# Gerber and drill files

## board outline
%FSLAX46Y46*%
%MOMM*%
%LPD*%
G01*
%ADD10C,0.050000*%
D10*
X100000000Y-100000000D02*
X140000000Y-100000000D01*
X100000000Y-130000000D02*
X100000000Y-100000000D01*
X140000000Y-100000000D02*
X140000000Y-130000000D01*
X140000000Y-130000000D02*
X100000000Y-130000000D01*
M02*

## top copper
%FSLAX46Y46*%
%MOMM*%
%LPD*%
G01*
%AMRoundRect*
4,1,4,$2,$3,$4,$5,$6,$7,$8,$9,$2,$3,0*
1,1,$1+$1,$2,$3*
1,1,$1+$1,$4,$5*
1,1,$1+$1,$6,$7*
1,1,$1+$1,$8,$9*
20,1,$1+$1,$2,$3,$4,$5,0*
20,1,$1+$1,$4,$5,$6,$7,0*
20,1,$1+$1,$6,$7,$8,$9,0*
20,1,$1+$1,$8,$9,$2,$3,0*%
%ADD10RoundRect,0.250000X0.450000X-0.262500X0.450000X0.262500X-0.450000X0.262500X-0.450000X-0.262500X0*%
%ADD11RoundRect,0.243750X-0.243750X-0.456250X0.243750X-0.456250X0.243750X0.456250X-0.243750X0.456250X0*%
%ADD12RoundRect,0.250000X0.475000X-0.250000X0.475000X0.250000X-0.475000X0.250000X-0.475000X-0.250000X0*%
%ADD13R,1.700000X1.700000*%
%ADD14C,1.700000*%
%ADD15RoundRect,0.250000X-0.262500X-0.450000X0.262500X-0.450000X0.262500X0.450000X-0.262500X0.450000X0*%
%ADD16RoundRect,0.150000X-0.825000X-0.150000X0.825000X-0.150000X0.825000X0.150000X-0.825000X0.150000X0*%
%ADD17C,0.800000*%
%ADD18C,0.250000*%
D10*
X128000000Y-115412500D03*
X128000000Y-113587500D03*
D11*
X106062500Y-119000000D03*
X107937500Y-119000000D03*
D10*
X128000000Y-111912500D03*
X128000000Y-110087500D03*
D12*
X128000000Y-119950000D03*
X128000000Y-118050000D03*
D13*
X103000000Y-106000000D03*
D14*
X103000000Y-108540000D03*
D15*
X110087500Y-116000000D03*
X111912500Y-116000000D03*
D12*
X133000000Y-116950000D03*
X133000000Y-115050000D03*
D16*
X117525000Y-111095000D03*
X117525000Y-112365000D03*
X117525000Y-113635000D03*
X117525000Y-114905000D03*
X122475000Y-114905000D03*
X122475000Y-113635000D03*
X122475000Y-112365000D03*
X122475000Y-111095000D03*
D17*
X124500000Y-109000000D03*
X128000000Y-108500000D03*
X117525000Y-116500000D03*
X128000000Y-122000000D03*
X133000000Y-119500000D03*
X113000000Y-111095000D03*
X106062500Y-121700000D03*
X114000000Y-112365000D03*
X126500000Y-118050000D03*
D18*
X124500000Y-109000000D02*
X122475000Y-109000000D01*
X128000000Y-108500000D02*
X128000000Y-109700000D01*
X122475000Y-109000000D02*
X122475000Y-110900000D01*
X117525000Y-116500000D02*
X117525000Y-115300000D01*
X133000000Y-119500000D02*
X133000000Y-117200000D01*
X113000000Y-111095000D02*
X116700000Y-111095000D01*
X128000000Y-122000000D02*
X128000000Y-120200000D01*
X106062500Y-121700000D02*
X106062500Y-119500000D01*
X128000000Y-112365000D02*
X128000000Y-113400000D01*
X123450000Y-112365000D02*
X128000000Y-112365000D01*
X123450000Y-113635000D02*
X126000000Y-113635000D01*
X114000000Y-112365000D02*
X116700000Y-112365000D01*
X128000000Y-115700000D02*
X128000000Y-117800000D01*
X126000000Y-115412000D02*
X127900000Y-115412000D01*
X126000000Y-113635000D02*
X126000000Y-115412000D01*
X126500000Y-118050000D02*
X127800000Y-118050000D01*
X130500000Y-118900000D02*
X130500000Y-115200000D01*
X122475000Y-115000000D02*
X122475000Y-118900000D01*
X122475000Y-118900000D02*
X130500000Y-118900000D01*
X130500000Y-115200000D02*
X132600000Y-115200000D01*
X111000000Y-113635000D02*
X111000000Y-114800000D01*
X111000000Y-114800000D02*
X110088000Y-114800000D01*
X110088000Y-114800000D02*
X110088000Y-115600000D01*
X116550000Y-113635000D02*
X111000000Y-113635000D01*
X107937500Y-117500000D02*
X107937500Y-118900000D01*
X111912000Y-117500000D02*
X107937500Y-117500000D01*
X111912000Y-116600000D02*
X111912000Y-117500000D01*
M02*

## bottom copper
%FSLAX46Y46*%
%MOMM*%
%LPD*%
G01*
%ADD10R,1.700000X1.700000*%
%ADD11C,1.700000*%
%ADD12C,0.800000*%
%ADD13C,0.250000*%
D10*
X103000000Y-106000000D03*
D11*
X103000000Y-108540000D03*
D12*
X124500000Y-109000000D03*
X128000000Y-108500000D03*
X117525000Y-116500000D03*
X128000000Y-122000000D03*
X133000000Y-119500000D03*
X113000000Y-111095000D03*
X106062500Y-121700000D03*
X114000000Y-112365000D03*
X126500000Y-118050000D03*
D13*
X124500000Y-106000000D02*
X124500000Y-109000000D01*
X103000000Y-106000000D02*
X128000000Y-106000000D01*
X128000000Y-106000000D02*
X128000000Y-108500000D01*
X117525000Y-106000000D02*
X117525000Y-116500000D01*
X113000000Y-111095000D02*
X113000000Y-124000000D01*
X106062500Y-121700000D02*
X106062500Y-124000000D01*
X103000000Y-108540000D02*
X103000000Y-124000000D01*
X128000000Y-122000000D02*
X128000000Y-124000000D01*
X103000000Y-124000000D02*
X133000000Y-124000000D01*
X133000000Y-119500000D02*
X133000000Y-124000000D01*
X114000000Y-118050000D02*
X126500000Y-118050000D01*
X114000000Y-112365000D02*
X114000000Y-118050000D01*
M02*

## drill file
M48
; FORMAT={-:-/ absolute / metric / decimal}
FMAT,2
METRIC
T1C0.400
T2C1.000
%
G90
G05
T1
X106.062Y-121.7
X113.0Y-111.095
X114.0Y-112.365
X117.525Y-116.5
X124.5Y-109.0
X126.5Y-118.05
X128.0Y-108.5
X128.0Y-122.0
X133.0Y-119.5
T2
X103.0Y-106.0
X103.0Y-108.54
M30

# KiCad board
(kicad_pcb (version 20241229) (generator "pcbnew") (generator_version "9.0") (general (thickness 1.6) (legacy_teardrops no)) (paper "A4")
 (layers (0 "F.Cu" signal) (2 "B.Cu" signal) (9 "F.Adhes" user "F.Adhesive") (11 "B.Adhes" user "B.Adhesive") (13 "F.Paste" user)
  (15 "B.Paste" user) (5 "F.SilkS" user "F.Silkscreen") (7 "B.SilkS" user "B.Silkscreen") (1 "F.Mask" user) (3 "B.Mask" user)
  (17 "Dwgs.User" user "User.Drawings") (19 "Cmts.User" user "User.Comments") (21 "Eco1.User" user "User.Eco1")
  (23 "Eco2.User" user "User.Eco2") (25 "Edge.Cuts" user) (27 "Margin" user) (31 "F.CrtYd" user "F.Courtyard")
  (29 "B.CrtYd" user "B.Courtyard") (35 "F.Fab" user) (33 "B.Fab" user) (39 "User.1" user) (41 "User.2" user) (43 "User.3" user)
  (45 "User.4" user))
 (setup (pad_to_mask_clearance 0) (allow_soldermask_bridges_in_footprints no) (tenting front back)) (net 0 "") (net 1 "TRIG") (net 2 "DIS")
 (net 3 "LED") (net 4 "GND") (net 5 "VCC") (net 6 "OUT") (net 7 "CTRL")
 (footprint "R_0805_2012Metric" (layer "F.Cu") (at 128 114.5 90)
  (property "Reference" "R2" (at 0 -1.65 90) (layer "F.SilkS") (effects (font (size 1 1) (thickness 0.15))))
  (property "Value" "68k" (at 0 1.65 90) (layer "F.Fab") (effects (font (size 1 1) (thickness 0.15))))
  (pad "1" smd roundrect (at -0.9125 0 90) (size 1.025 1.4) (layers "F.Cu" "F.Mask" "F.Paste") (roundrect_rratio 0.243902) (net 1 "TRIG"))
  (pad "2" smd roundrect (at 0.9125 0 90) (size 1.025 1.4) (layers "F.Cu" "F.Mask" "F.Paste") (roundrect_rratio 0.243902) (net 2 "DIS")))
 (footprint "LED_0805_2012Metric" (layer "F.Cu") (at 107 119)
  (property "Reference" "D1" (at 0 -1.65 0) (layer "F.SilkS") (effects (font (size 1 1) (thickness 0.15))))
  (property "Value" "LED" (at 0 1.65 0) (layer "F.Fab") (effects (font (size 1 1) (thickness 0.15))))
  (pad "1" smd roundrect (at -0.9375 0) (size 0.975 1.4) (layers "F.Cu" "F.Mask" "F.Paste") (roundrect_rratio 0.25) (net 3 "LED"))
  (pad "2" smd roundrect (at 0.9375 0) (size 0.975 1.4) (layers "F.Cu" "F.Mask" "F.Paste") (roundrect_rratio 0.25) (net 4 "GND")))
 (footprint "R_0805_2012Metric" (layer "F.Cu") (at 128 111 90)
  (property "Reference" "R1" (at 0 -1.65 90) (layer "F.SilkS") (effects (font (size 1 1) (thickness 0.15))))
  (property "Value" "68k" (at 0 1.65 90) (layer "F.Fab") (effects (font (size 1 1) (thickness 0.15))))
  (pad "1" smd roundrect (at -0.9125 0 90) (size 1.025 1.4) (layers "F.Cu" "F.Mask" "F.Paste") (roundrect_rratio 0.243902) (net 2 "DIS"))
  (pad "2" smd roundrect (at 0.9125 0 90) (size 1.025 1.4) (layers "F.Cu" "F.Mask" "F.Paste") (roundrect_rratio 0.243902) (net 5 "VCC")))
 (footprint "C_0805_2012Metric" (layer "F.Cu") (at 128 119 90)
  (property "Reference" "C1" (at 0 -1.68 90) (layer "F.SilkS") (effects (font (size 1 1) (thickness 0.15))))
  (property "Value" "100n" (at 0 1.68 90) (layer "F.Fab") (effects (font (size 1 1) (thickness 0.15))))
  (pad "1" smd roundrect (at -0.95 0 90) (size 1 1.45) (layers "F.Cu" "F.Mask" "F.Paste") (roundrect_rratio 0.25) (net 4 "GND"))
  (pad "2" smd roundrect (at 0.95 0 90) (size 1 1.45) (layers "F.Cu" "F.Mask" "F.Paste") (roundrect_rratio 0.25) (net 1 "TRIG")))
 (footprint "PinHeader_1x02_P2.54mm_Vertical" (layer "F.Cu") (at 103 106)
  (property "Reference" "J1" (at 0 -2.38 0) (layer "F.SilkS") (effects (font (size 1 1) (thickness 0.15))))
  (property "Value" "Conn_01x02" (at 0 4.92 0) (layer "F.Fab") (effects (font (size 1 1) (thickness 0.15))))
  (pad "1" thru_hole rect (at 0 0) (size 1.7 1.7) (drill 1) (layers "*.Cu" "*.Mask") (remove_unused_layers no) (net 5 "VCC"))
  (pad "2" thru_hole circle (at 0 2.54) (size 1.7 1.7) (drill 1) (layers "*.Cu" "*.Mask") (remove_unused_layers no) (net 4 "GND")))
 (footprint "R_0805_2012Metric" (layer "F.Cu") (at 111 116)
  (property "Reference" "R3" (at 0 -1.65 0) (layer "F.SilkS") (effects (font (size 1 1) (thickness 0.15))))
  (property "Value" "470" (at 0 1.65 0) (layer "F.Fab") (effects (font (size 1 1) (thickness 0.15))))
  (pad "1" smd roundrect (at -0.9125 0) (size 1.025 1.4) (layers "F.Cu" "F.Mask" "F.Paste") (roundrect_rratio 0.243902) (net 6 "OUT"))
  (pad "2" smd roundrect (at 0.9125 0) (size 1.025 1.4) (layers "F.Cu" "F.Mask" "F.Paste") (roundrect_rratio 0.243902) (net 3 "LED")))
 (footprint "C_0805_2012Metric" (layer "F.Cu") (at 133 116 90)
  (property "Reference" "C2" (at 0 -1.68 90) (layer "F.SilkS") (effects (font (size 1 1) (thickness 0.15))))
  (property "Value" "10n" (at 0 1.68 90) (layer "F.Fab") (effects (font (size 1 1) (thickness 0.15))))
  (pad "1" smd roundrect (at -0.95 0 90) (size 1 1.45) (layers "F.Cu" "F.Mask" "F.Paste") (roundrect_rratio 0.25) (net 4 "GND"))
  (pad "2" smd roundrect (at 0.95 0 90) (size 1 1.45) (layers "F.Cu" "F.Mask" "F.Paste") (roundrect_rratio 0.25) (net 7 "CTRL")))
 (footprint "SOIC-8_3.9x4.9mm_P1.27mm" (layer "F.Cu") (at 120 113)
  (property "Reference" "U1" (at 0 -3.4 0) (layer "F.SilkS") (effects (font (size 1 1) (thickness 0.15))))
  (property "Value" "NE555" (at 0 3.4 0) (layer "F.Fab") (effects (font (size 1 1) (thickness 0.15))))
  (pad "1" smd roundrect (at -2.475 -1.905) (size 1.95 0.6) (layers "F.Cu" "F.Mask" "F.Paste") (roundrect_rratio 0.25) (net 4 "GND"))
  (pad "2" smd roundrect (at -2.475 -0.635) (size 1.95 0.6) (layers "F.Cu" "F.Mask" "F.Paste") (roundrect_rratio 0.25) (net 1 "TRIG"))
  (pad "3" smd roundrect (at -2.475 0.635) (size 1.95 0.6) (layers "F.Cu" "F.Mask" "F.Paste") (roundrect_rratio 0.25) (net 6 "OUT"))
  (pad "4" smd roundrect (at -2.475 1.905) (size 1.95 0.6) (layers "F.Cu" "F.Mask" "F.Paste") (roundrect_rratio 0.25) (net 5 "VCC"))
  (pad "5" smd roundrect (at 2.475 1.905) (size 1.95 0.6) (layers "F.Cu" "F.Mask" "F.Paste") (roundrect_rratio 0.25) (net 7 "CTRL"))
  (pad "6" smd roundrect (at 2.475 0.635) (size 1.95 0.6) (layers "F.Cu" "F.Mask" "F.Paste") (roundrect_rratio 0.25) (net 1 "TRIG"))
  (pad "7" smd roundrect (at 2.475 -0.635) (size 1.95 0.6) (layers "F.Cu" "F.Mask" "F.Paste") (roundrect_rratio 0.25) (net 2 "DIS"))
  (pad "8" smd roundrect (at 2.475 -1.905) (size 1.95 0.6) (layers "F.Cu" "F.Mask" "F.Paste") (roundrect_rratio 0.25) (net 5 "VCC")))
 (gr_line (start 100 100) (end 140 100) (stroke (width 0.05) (type default)) (layer "Edge.Cuts"))
 (gr_line (start 100 130) (end 100 100) (stroke (width 0.05) (type default)) (layer "Edge.Cuts"))
 (gr_line (start 140 100) (end 140 130) (stroke (width 0.05) (type default)) (layer "Edge.Cuts"))
 (gr_line (start 140 130) (end 100 130) (stroke (width 0.05) (type default)) (layer "Edge.Cuts"))
 (segment (start 124.5 109) (end 122.475 109) (width 0.25) (layer "F.Cu") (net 5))
 (segment (start 128 108.5) (end 128 109.7) (width 0.25) (layer "F.Cu") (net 5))
 (segment (start 122.475 109) (end 122.475 110.9) (width 0.25) (layer "F.Cu") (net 5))
 (segment (start 117.525 116.5) (end 117.525 115.3) (width 0.25) (layer "F.Cu") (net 5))
 (via (at 124.5 109) (size 0.8) (drill 0.4) (layers "F.Cu" "B.Cu") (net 5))
 (via (at 128 108.5) (size 0.8) (drill 0.4) (layers "F.Cu" "B.Cu") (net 5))
 (via (at 117.525 116.5) (size 0.8) (drill 0.4) (layers "F.Cu" "B.Cu") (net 5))
 (segment (start 124.5 106) (end 124.5 109) (width 0.25) (layer "B.Cu") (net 5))
 (segment (start 103 106) (end 128 106) (width 0.25) (layer "B.Cu") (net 5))
 (segment (start 128 106) (end 128 108.5) (width 0.25) (layer "B.Cu") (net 5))
 (segment (start 117.525 106) (end 117.525 116.5) (width 0.25) (layer "B.Cu") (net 5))
 (segment (start 133 119.5) (end 133 117.2) (width 0.25) (layer "F.Cu") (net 4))
 (segment (start 113 111.095) (end 116.7 111.095) (width 0.25) (layer "F.Cu") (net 4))
 (segment (start 128 122) (end 128 120.2) (width 0.25) (layer "F.Cu") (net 4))
 (segment (start 106.0625 121.7) (end 106.0625 119.5) (width 0.25) (layer "F.Cu") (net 4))
 (via (at 128 122) (size 0.8) (drill 0.4) (layers "F.Cu" "B.Cu") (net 4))
 (via (at 133 119.5) (size 0.8) (drill 0.4) (layers "F.Cu" "B.Cu") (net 4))
 (via (at 113 111.095) (size 0.8) (drill 0.4) (layers "F.Cu" "B.Cu") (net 4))
 (via (at 106.0625 121.7) (size 0.8) (drill 0.4) (layers "F.Cu" "B.Cu") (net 4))
 (segment (start 113 111.095) (end 113 124) (width 0.25) (layer "B.Cu") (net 4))
 (segment (start 106.0625 121.7) (end 106.0625 124) (width 0.25) (layer "B.Cu") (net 4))
 (segment (start 103 108.54) (end 103 124) (width 0.25) (layer "B.Cu") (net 4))
 (segment (start 128 122) (end 128 124) (width 0.25) (layer "B.Cu") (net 4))
 (segment (start 103 124) (end 133 124) (width 0.25) (layer "B.Cu") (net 4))
 (segment (start 133 119.5) (end 133 124) (width 0.25) (layer "B.Cu") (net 4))
 (segment (start 128 112.365) (end 128 113.4) (width 0.25) (layer "F.Cu") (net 2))
 (segment (start 123.45 112.365) (end 128 112.365) (width 0.25) (layer "F.Cu") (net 2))
 (segment (start 123.45 113.635) (end 126 113.635) (width 0.25) (layer "F.Cu") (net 1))
 (segment (start 114 112.365) (end 116.7 112.365) (width 0.25) (layer "F.Cu") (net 1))
 (segment (start 128 115.7) (end 128 117.8) (width 0.25) (layer "F.Cu") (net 1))
 (segment (start 126 115.412) (end 127.9 115.412) (width 0.25) (layer "F.Cu") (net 1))
 (segment (start 126 113.635) (end 126 115.412) (width 0.25) (layer "F.Cu") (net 1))
 (segment (start 126.5 118.05) (end 127.8 118.05) (width 0.25) (layer "F.Cu") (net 1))
 (via (at 114 112.365) (size 0.8) (drill 0.4) (layers "F.Cu" "B.Cu") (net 1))
 (via (at 126.5 118.05) (size 0.8) (drill 0.4) (layers "F.Cu" "B.Cu") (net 1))
 (segment (start 114 118.05) (end 126.5 118.05) (width 0.25) (layer "B.Cu") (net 1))
 (segment (start 114 112.365) (end 114 118.05) (width 0.25) (layer "B.Cu") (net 1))
 (segment (start 130.5 118.9) (end 130.5 115.2) (width 0.25) (layer "F.Cu") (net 7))
 (segment (start 122.475 115) (end 122.475 118.9) (width 0.25) (layer "F.Cu") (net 7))
 (segment (start 122.475 118.9) (end 130.5 118.9) (width 0.25) (layer "F.Cu") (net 7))
 (segment (start 130.5 115.2) (end 132.6 115.2) (width 0.25) (layer "F.Cu") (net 7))
 (segment (start 111 113.635) (end 111 114.8) (width 0.25) (layer "F.Cu") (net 6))
 (segment (start 111 114.8) (end 110.088 114.8) (width 0.25) (layer "F.Cu") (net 6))
 (segment (start 110.088 114.8) (end 110.088 115.6) (width 0.25) (layer "F.Cu") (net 6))
 (segment (start 116.55 113.635) (end 111 113.635) (width 0.25) (layer "F.Cu") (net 6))
 (segment (start 107.9375 117.5) (end 107.9375 118.9) (width 0.25) (layer "F.Cu") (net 3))
 (segment (start 111.912 117.5) (end 107.9375 117.5) (width 0.25) (layer "F.Cu") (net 3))
 (segment (start 111.912 116.6) (end 111.912 117.5) (width 0.25) (layer "F.Cu") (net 3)))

